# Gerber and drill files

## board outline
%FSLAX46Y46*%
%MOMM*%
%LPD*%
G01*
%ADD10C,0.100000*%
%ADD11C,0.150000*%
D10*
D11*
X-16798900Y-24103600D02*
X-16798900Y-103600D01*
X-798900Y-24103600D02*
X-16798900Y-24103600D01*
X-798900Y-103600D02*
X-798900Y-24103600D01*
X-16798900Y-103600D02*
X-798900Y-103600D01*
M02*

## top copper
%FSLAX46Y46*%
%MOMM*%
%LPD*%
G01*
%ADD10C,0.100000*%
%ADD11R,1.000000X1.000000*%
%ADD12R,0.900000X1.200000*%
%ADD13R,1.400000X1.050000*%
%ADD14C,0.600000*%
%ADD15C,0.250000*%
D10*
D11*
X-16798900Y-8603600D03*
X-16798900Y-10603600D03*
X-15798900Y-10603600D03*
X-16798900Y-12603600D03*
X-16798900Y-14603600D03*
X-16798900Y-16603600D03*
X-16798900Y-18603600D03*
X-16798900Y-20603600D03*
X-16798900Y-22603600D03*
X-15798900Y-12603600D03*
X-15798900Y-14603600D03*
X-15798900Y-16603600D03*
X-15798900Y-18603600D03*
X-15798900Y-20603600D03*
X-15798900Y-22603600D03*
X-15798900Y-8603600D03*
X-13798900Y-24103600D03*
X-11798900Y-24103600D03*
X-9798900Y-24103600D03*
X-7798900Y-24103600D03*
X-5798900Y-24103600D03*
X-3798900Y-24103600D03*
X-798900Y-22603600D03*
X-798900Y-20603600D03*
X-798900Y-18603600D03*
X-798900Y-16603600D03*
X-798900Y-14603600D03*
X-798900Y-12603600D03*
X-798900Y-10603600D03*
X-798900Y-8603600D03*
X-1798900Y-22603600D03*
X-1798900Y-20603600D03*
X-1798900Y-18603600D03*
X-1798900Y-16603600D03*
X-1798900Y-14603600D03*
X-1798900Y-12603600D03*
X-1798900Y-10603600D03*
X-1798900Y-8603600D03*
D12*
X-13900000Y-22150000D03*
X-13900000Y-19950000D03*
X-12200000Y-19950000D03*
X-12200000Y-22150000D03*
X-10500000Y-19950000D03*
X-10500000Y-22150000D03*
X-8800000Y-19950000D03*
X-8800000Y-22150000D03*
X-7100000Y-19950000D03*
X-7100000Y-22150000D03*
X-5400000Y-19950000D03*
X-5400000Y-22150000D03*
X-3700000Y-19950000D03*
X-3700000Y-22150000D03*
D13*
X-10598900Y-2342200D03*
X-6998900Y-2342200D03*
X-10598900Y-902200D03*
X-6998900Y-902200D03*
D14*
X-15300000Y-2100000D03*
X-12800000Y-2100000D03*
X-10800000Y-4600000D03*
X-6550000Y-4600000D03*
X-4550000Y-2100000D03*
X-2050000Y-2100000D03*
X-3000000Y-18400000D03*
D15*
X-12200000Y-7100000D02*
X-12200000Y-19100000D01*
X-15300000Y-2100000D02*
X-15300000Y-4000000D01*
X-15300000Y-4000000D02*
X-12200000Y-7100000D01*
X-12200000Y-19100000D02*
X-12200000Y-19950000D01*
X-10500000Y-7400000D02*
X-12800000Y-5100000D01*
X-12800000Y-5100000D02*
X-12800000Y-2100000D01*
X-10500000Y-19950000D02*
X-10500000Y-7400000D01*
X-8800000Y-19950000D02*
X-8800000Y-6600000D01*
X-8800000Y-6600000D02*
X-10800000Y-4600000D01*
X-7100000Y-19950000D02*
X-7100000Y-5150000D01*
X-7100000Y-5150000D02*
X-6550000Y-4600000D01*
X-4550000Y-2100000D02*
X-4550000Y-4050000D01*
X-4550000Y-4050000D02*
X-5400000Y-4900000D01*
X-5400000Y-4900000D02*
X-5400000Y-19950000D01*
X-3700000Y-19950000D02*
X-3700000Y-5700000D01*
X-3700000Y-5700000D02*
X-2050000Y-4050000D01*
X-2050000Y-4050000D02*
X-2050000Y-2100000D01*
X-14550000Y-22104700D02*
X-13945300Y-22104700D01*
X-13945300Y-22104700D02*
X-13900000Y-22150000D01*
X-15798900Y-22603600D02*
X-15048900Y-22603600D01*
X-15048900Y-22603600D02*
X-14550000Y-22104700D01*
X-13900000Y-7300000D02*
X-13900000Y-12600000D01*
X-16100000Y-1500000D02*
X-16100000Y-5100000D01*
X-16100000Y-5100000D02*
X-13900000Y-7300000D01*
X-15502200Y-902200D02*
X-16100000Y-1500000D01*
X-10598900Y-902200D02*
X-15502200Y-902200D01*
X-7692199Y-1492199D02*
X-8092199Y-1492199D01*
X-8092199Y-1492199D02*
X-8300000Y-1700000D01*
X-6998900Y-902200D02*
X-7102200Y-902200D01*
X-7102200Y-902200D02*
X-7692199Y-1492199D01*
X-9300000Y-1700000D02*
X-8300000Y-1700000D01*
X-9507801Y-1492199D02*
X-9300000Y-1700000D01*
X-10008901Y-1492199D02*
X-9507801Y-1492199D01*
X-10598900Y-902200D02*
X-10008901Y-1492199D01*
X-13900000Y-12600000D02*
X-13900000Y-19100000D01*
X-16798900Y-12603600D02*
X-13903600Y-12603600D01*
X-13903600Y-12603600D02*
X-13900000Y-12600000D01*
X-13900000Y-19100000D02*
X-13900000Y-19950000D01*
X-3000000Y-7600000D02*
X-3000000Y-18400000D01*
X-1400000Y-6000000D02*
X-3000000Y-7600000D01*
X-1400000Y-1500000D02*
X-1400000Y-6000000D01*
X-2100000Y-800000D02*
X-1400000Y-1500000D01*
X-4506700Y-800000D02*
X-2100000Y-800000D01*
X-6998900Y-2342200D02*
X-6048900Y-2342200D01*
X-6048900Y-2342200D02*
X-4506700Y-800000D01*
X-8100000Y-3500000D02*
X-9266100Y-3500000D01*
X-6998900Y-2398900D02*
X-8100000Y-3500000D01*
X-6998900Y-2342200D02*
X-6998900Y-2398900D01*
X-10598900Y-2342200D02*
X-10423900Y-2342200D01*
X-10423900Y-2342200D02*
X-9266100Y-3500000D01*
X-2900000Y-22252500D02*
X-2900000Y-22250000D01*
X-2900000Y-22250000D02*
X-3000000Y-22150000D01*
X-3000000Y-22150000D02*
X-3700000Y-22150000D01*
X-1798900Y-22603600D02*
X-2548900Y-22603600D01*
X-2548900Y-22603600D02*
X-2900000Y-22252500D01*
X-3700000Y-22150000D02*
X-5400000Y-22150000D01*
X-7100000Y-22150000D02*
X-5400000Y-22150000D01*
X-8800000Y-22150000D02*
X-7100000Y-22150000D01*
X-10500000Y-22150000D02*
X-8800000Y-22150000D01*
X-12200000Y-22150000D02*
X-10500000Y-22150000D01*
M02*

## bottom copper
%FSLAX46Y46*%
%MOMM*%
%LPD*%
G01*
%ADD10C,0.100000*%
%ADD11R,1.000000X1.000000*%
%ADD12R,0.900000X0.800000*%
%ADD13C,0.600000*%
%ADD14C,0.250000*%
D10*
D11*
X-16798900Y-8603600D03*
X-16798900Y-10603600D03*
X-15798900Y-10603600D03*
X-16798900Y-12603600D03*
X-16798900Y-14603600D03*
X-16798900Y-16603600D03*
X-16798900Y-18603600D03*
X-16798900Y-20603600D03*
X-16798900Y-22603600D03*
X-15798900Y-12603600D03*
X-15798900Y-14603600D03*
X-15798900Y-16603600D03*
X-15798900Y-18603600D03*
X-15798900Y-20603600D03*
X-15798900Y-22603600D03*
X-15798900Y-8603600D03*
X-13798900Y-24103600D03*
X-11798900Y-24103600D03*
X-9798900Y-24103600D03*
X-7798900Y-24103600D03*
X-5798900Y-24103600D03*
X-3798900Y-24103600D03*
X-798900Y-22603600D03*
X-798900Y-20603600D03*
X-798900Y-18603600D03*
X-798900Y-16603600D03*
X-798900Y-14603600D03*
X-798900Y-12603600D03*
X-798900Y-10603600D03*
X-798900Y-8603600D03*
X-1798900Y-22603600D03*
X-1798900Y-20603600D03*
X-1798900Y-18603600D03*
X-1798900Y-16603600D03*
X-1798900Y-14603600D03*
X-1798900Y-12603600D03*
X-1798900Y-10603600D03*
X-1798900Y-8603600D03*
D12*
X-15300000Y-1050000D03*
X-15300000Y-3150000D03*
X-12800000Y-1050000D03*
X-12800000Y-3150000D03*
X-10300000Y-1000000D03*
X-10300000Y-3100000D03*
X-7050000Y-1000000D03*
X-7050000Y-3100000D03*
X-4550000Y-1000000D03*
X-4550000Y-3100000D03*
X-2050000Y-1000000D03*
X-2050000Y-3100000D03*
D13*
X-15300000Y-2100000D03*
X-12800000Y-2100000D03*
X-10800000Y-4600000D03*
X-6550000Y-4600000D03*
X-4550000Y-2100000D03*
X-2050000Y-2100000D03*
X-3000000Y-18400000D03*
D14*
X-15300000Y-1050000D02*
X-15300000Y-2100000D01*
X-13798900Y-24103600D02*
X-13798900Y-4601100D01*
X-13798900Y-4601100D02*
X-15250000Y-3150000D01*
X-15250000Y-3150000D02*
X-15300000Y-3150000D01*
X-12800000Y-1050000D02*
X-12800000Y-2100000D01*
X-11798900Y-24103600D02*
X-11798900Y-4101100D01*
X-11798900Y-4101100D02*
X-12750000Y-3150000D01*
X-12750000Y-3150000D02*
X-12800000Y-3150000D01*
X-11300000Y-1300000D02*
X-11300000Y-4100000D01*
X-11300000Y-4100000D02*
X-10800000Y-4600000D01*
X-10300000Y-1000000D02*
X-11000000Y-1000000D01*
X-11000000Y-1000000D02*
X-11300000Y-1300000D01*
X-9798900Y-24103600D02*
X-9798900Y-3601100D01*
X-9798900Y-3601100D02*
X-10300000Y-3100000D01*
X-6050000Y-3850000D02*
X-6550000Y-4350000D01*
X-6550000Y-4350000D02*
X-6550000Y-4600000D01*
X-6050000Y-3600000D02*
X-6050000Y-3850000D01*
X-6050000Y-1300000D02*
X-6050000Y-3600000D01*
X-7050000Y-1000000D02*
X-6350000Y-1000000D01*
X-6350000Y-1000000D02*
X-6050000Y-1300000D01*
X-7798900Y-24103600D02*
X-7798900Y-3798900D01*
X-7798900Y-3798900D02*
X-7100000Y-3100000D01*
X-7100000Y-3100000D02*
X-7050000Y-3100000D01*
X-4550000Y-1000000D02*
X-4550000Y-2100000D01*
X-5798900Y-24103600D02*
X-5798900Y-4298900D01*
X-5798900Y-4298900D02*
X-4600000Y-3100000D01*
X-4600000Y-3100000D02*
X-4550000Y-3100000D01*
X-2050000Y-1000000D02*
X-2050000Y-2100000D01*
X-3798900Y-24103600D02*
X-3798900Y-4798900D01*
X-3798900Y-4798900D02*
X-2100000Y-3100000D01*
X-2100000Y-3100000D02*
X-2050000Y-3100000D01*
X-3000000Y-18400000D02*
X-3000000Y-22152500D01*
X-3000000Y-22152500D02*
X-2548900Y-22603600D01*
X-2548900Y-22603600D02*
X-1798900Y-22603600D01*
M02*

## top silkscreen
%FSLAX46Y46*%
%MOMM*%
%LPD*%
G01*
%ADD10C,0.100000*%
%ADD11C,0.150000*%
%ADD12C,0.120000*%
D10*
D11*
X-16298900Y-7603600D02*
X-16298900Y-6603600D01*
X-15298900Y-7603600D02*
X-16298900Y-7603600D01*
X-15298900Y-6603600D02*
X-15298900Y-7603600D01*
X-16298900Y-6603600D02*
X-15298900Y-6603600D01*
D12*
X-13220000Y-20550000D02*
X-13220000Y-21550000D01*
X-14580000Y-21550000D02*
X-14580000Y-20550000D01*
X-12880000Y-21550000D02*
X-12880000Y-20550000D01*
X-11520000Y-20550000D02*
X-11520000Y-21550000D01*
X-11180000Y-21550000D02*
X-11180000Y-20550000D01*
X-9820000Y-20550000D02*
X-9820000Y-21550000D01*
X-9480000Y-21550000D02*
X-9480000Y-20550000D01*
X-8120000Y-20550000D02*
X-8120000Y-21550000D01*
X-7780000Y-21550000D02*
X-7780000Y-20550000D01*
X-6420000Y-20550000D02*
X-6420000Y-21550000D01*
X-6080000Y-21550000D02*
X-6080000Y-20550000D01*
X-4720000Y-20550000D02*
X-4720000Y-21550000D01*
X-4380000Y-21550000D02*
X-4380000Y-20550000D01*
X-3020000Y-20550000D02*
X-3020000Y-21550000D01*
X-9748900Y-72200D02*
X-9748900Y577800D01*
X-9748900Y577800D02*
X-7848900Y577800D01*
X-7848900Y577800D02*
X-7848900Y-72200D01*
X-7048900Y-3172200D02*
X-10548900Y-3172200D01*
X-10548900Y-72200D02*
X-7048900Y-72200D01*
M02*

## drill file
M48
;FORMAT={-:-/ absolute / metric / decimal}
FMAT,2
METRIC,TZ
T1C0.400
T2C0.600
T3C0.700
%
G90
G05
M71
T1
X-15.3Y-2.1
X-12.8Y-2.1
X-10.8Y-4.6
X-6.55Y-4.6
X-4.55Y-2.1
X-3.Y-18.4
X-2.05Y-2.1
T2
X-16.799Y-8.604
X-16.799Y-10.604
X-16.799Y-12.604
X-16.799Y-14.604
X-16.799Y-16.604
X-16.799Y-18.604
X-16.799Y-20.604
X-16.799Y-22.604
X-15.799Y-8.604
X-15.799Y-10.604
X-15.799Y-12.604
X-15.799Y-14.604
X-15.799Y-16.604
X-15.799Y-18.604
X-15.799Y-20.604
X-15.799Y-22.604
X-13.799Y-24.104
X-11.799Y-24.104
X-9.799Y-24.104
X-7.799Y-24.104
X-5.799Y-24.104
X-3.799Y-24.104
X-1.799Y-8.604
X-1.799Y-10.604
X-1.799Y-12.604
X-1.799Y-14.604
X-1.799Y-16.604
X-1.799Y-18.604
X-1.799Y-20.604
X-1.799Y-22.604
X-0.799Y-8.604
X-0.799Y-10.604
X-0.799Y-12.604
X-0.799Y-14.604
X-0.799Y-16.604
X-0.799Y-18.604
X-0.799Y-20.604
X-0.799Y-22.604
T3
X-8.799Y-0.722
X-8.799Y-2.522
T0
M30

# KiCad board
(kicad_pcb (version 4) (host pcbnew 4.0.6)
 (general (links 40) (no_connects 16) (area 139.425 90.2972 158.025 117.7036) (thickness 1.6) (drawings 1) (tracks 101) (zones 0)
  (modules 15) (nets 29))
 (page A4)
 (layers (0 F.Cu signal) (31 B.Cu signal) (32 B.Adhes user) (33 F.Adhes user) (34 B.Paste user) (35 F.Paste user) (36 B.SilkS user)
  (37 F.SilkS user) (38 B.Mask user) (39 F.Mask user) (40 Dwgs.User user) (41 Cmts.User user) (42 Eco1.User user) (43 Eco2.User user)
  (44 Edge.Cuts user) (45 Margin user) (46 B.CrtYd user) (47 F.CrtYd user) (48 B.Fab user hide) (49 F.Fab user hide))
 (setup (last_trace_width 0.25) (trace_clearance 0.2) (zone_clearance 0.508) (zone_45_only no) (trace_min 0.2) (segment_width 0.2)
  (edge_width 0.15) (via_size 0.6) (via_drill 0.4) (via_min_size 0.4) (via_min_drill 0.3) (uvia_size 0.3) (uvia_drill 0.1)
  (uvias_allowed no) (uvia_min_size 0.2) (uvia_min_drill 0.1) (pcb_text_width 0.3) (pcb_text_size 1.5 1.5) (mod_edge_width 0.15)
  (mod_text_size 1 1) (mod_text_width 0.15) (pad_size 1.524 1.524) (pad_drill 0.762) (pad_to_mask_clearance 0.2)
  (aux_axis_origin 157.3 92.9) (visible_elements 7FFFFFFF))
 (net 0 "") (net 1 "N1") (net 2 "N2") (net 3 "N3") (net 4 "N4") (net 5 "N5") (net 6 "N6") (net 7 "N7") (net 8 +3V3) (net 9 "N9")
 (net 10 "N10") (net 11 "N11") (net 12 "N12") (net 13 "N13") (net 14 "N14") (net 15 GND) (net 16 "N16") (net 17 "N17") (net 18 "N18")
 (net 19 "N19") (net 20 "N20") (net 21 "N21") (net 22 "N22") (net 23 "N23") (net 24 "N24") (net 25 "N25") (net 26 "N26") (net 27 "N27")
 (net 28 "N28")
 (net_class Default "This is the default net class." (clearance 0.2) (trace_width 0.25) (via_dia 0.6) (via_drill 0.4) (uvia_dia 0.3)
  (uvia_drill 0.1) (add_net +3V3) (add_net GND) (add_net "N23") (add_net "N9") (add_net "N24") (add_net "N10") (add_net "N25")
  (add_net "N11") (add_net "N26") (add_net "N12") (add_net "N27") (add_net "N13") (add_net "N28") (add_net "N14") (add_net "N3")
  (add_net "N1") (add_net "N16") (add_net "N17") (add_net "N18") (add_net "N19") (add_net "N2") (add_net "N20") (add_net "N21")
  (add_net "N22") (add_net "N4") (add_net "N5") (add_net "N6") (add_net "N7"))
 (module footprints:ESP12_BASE (layer F.Cu) (at 148.5011 105.0036)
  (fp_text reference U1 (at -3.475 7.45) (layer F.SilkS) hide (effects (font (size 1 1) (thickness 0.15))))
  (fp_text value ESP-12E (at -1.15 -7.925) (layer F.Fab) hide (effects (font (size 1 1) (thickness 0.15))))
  (fp_line (start -7.5 -4.5) (end -7.5 -5.5) (layer F.SilkS) (width 0.15))
  (fp_line (start -6.5 -4.5) (end -7.5 -4.5) (layer F.SilkS) (width 0.15))
  (fp_line (start -6.5 -5.5) (end -6.5 -4.5) (layer F.SilkS) (width 0.15))
  (fp_line (start -7.5 -5.5) (end -6.5 -5.5) (layer F.SilkS) (width 0.15))
  (fp_line (start -8 12) (end -8 -12) (layer Edge.Cuts) (width 0.15))
  (fp_line (start 8 12) (end -8 12) (layer Edge.Cuts) (width 0.15))
  (fp_line (start 8 -12) (end 8 12) (layer Edge.Cuts) (width 0.15))
  (fp_line (start -8 -12) (end 8 -12) (layer Edge.Cuts) (width 0.15))
  (pad 1 thru_hole rect (at -8 -3.5) (size 1 1) (drill 0.6) (layers *.Cu *.Mask) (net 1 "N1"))
  (pad 2 thru_hole rect (at -8 -1.5) (size 1 1) (drill 0.6) (layers *.Cu *.Mask) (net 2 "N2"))
  (pad 2 thru_hole rect (at -7 -1.5) (size 1 1) (drill 0.6) (layers *.Cu *.Mask) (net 2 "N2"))
  (pad 3 thru_hole rect (at -8 0.5) (size 1 1) (drill 0.6) (layers *.Cu *.Mask) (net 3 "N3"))
  (pad 4 thru_hole rect (at -8 2.5) (size 1 1) (drill 0.6) (layers *.Cu *.Mask) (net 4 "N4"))
  (pad 5 thru_hole rect (at -8 4.5) (size 1 1) (drill 0.6) (layers *.Cu *.Mask) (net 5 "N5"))
  (pad 6 thru_hole rect (at -8 6.5) (size 1 1) (drill 0.6) (layers *.Cu *.Mask) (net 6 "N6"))
  (pad 7 thru_hole rect (at -8 8.5) (size 1 1) (drill 0.6) (layers *.Cu *.Mask) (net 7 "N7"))
  (pad 8 thru_hole rect (at -8 10.5) (size 1 1) (drill 0.6) (layers *.Cu *.Mask) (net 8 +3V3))
  (pad 3 thru_hole rect (at -7 0.5) (size 1 1) (drill 0.6) (layers *.Cu *.Mask) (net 3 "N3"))
  (pad 4 thru_hole rect (at -7 2.5) (size 1 1) (drill 0.6) (layers *.Cu *.Mask) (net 4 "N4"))
  (pad 5 thru_hole rect (at -7 4.5) (size 1 1) (drill 0.6) (layers *.Cu *.Mask) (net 5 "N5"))
  (pad 6 thru_hole rect (at -7 6.5) (size 1 1) (drill 0.6) (layers *.Cu *.Mask) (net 6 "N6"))
  (pad 7 thru_hole rect (at -7 8.5) (size 1 1) (drill 0.6) (layers *.Cu *.Mask) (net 7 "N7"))
  (pad 8 thru_hole rect (at -7 10.5) (size 1 1) (drill 0.6) (layers *.Cu *.Mask) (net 8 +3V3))
  (pad 1 thru_hole rect (at -7 -3.5) (size 1 1) (drill 0.6) (layers *.Cu *.Mask) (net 1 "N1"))
  (pad 9 thru_hole rect (at -5 12) (size 1 1) (drill 0.6) (layers *.Cu *.Mask) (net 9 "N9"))
  (pad 10 thru_hole rect (at -3 12) (size 1 1) (drill 0.6) (layers *.Cu *.Mask) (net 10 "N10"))
  (pad 11 thru_hole rect (at -1 12) (size 1 1) (drill 0.6) (layers *.Cu *.Mask) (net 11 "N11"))
  (pad 12 thru_hole rect (at 1 12) (size 1 1) (drill 0.6) (layers *.Cu *.Mask) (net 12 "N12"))
  (pad 13 thru_hole rect (at 3 12) (size 1 1) (drill 0.6) (layers *.Cu *.Mask) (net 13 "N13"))
  (pad 14 thru_hole rect (at 5 12) (size 1 1) (drill 0.6) (layers *.Cu *.Mask) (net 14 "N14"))
  (pad 15 thru_hole rect (at 8 10.5) (size 1 1) (drill 0.6) (layers *.Cu *.Mask) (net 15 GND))
  (pad 16 thru_hole rect (at 8 8.5) (size 1 1) (drill 0.6) (layers *.Cu *.Mask) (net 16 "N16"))
  (pad 17 thru_hole rect (at 8 6.5) (size 1 1) (drill 0.6) (layers *.Cu *.Mask) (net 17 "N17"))
  (pad 18 thru_hole rect (at 8 4.5) (size 1 1) (drill 0.6) (layers *.Cu *.Mask) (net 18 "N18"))
  (pad 19 thru_hole rect (at 8 2.5) (size 1 1) (drill 0.6) (layers *.Cu *.Mask) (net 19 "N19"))
  (pad 20 thru_hole rect (at 8 0.5) (size 1 1) (drill 0.6) (layers *.Cu *.Mask) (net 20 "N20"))
  (pad 21 thru_hole rect (at 8 -1.5) (size 1 1) (drill 0.6) (layers *.Cu *.Mask) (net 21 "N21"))
  (pad 22 thru_hole rect (at 8 -3.5) (size 1 1) (drill 0.6) (layers *.Cu *.Mask) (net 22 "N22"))
  (pad 15 thru_hole rect (at 7 10.5) (size 1 1) (drill 0.6) (layers *.Cu *.Mask) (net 15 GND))
  (pad 16 thru_hole rect (at 7 8.5) (size 1 1) (drill 0.6) (layers *.Cu *.Mask) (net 16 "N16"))
  (pad 17 thru_hole rect (at 7 6.5) (size 1 1) (drill 0.6) (layers *.Cu *.Mask) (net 17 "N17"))
  (pad 18 thru_hole rect (at 7 4.5) (size 1 1) (drill 0.6) (layers *.Cu *.Mask) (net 18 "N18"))
  (pad 19 thru_hole rect (at 7 2.5) (size 1 1) (drill 0.6) (layers *.Cu *.Mask) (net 19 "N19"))
  (pad 20 thru_hole rect (at 7 0.5) (size 1 1) (drill 0.6) (layers *.Cu *.Mask) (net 20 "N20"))
  (pad 21 thru_hole rect (at 7 -1.5) (size 1 1) (drill 0.6) (layers *.Cu *.Mask) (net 21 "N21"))
  (pad 22 thru_hole rect (at 7 -3.5) (size 1 1) (drill 0.6) (layers *.Cu *.Mask) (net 22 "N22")))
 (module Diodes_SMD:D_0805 (layer B.Cu) (at 142 95 270)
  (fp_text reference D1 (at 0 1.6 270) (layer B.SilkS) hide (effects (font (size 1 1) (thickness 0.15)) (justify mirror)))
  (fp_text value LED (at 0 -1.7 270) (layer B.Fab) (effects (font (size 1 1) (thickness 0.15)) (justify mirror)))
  (pad 1 smd rect (at -1.05 0 270) (size 0.8 0.9) (layers B.Cu B.Paste B.Mask) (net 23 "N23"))
  (pad 2 smd rect (at 1.05 0 270) (size 0.8 0.9) (layers B.Cu B.Paste B.Mask) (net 9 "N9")))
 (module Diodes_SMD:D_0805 (layer B.Cu) (at 144.5 95 270)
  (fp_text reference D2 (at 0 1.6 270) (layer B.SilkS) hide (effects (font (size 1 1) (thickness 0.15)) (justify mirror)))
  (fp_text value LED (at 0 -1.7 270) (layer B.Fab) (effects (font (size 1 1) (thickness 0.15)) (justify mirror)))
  (pad 1 smd rect (at -1.05 0 270) (size 0.8 0.9) (layers B.Cu B.Paste B.Mask) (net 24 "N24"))
  (pad 2 smd rect (at 1.05 0 270) (size 0.8 0.9) (layers B.Cu B.Paste B.Mask) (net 10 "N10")))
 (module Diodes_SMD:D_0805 (layer B.Cu) (at 147 94.95 270)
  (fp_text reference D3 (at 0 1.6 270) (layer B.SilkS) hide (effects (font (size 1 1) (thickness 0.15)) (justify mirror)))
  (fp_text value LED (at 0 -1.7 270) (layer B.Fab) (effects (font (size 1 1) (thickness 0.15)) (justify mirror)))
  (pad 1 smd rect (at -1.05 0 270) (size 0.8 0.9) (layers B.Cu B.Paste B.Mask) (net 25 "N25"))
  (pad 2 smd rect (at 1.05 0 270) (size 0.8 0.9) (layers B.Cu B.Paste B.Mask) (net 11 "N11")))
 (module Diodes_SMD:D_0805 (layer B.Cu) (at 150.25 94.95 270)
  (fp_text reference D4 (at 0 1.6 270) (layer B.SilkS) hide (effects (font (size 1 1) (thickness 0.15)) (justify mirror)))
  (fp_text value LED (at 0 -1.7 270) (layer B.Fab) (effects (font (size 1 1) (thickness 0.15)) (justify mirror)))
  (pad 1 smd rect (at -1.05 0 270) (size 0.8 0.9) (layers B.Cu B.Paste B.Mask) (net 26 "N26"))
  (pad 2 smd rect (at 1.05 0 270) (size 0.8 0.9) (layers B.Cu B.Paste B.Mask) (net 12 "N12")))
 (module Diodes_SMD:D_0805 (layer B.Cu) (at 152.75 94.95 270)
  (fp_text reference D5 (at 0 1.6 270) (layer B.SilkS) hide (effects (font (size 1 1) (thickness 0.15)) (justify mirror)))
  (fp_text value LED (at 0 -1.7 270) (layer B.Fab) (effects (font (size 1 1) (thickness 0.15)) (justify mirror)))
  (pad 1 smd rect (at -1.05 0 270) (size 0.8 0.9) (layers B.Cu B.Paste B.Mask) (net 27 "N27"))
  (pad 2 smd rect (at 1.05 0 270) (size 0.8 0.9) (layers B.Cu B.Paste B.Mask) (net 13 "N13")))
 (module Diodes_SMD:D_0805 (layer B.Cu) (at 155.25 94.95 270)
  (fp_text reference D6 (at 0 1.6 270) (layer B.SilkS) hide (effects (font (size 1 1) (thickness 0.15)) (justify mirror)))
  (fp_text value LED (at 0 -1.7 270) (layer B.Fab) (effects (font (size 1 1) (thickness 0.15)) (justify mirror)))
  (pad 1 smd rect (at -1.05 0 270) (size 0.8 0.9) (layers B.Cu B.Paste B.Mask) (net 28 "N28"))
  (pad 2 smd rect (at 1.05 0 270) (size 0.8 0.9) (layers B.Cu B.Paste B.Mask) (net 14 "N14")))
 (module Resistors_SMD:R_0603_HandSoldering (layer F.Cu) (at 143.4 113.95 90)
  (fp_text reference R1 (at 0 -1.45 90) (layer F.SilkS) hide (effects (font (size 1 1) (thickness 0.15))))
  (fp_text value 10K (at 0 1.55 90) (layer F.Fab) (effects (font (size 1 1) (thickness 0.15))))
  (fp_line (start 0.5 0.68) (end -0.5 0.68) (layer F.SilkS) (width 0.12))
  (fp_line (start -0.5 -0.68) (end 0.5 -0.68) (layer F.SilkS) (width 0.12))
  (pad 1 smd rect (at -1.1 0 90) (size 1.2 0.9) (layers F.Cu F.Paste F.Mask) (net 8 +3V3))
  (pad 2 smd rect (at 1.1 0 90) (size 1.2 0.9) (layers F.Cu F.Paste F.Mask) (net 3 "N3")))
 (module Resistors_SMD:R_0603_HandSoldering (layer F.Cu) (at 145.1 113.95 270)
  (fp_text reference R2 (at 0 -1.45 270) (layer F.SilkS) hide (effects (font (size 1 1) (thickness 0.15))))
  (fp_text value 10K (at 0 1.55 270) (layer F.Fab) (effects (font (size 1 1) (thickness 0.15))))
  (fp_line (start 0.5 0.68) (end -0.5 0.68) (layer F.SilkS) (width 0.12))
  (fp_line (start -0.5 -0.68) (end 0.5 -0.68) (layer F.SilkS) (width 0.12))
  (pad 1 smd rect (at -1.1 0 270) (size 1.2 0.9) (layers F.Cu F.Paste F.Mask) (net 23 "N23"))
  (pad 2 smd rect (at 1.1 0 270) (size 1.2 0.9) (layers F.Cu F.Paste F.Mask) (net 15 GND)))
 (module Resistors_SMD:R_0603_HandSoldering (layer F.Cu) (at 146.8 113.95 270)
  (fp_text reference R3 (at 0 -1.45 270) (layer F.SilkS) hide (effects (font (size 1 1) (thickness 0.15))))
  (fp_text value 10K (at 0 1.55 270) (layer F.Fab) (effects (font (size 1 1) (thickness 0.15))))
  (fp_line (start 0.5 0.68) (end -0.5 0.68) (layer F.SilkS) (width 0.12))
  (fp_line (start -0.5 -0.68) (end 0.5 -0.68) (layer F.SilkS) (width 0.12))
  (pad 1 smd rect (at -1.1 0 270) (size 1.2 0.9) (layers F.Cu F.Paste F.Mask) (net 24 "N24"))
  (pad 2 smd rect (at 1.1 0 270) (size 1.2 0.9) (layers F.Cu F.Paste F.Mask) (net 15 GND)))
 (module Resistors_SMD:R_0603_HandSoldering (layer F.Cu) (at 148.5 113.95 270)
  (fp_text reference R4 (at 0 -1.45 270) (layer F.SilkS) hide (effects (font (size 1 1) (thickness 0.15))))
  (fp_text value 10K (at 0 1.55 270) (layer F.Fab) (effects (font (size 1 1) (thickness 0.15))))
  (fp_line (start 0.5 0.68) (end -0.5 0.68) (layer F.SilkS) (width 0.12))
  (fp_line (start -0.5 -0.68) (end 0.5 -0.68) (layer F.SilkS) (width 0.12))
  (pad 1 smd rect (at -1.1 0 270) (size 1.2 0.9) (layers F.Cu F.Paste F.Mask) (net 25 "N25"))
  (pad 2 smd rect (at 1.1 0 270) (size 1.2 0.9) (layers F.Cu F.Paste F.Mask) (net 15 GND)))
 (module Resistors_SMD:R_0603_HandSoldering (layer F.Cu) (at 150.2 113.95 270)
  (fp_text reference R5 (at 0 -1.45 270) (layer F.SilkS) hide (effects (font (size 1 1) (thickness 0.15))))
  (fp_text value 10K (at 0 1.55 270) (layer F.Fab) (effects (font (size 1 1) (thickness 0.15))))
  (fp_line (start 0.5 0.68) (end -0.5 0.68) (layer F.SilkS) (width 0.12))
  (fp_line (start -0.5 -0.68) (end 0.5 -0.68) (layer F.SilkS) (width 0.12))
  (pad 1 smd rect (at -1.1 0 270) (size 1.2 0.9) (layers F.Cu F.Paste F.Mask) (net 26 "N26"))
  (pad 2 smd rect (at 1.1 0 270) (size 1.2 0.9) (layers F.Cu F.Paste F.Mask) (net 15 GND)))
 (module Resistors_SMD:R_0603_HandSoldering (layer F.Cu) (at 151.9 113.95 270)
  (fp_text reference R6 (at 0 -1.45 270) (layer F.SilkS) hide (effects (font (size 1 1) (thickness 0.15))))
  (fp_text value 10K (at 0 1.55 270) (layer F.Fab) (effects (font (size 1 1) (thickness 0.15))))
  (fp_line (start 0.5 0.68) (end -0.5 0.68) (layer F.SilkS) (width 0.12))
  (fp_line (start -0.5 -0.68) (end 0.5 -0.68) (layer F.SilkS) (width 0.12))
  (pad 1 smd rect (at -1.1 0 270) (size 1.2 0.9) (layers F.Cu F.Paste F.Mask) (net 27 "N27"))
  (pad 2 smd rect (at 1.1 0 270) (size 1.2 0.9) (layers F.Cu F.Paste F.Mask) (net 15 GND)))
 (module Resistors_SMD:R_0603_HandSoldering (layer F.Cu) (at 153.6 113.95 270)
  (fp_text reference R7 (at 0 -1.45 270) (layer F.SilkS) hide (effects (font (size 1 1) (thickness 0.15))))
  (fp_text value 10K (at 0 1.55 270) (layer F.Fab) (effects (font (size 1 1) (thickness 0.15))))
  (fp_line (start 0.5 0.68) (end -0.5 0.68) (layer F.SilkS) (width 0.12))
  (fp_line (start -0.5 -0.68) (end 0.5 -0.68) (layer F.SilkS) (width 0.12))
  (pad 1 smd rect (at -1.1 0 270) (size 1.2 0.9) (layers F.Cu F.Paste F.Mask) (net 28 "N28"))
  (pad 2 smd rect (at 1.1 0 270) (size 1.2 0.9) (layers F.Cu F.Paste F.Mask) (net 15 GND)))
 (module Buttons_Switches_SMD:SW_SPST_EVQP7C (layer F.Cu) (at 148.5011 94.5222 180)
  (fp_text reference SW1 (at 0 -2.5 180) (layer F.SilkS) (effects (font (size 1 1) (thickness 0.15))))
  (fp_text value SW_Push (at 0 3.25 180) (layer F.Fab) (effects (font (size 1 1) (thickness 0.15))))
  (fp_line (start 0.95 1.55) (end 0.95 2.2) (layer F.SilkS) (width 0.12))
  (fp_line (start 0.95 2.2) (end -0.95 2.2) (layer F.SilkS) (width 0.12))
  (fp_line (start -0.95 2.2) (end -0.95 1.55) (layer F.SilkS) (width 0.12))
  (fp_line (start -1.75 -1.55) (end 1.75 -1.55) (layer F.SilkS) (width 0.12))
  (fp_line (start 1.75 1.55) (end -1.75 1.55) (layer F.SilkS) (width 0.12))
  (pad 1 smd rect (at 1.8 -0.72 180) (size 1.4 1.05) (layers F.Cu F.Paste F.Mask) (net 15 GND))
  (pad 1 smd rect (at -1.8 -0.72 180) (size 1.4 1.05) (layers F.Cu F.Paste F.Mask) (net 15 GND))
  (pad 2 smd rect (at 1.8 0.72 180) (size 1.4 1.05) (layers F.Cu F.Paste F.Mask) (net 3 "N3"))
  (pad 2 smd rect (at -1.8 0.72 180) (size 1.4 1.05) (layers F.Cu F.Paste F.Mask) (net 3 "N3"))
  (pad "" np_thru_hole circle (at 0 -0.9 180) (size 0.7 0.7) (drill 0.7) (layers *.Cu *.Mask))
  (pad "" np_thru_hole circle (at 0 0.9 180) (size 0.7 0.7) (drill 0.7) (layers *.Cu *.Mask)))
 (segment (start 145.1 100) (end 145.1 112) (width 0.25) (layer F.Cu) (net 23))
 (segment (start 142 95) (end 142 96.9) (width 0.25) (layer F.Cu) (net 23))
 (segment (start 142 96.9) (end 145.1 100) (width 0.25) (layer F.Cu) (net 23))
 (segment (start 145.1 112) (end 145.1 112.85) (width 0.25) (layer F.Cu) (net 23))
 (segment (start 142 93.95) (end 142 95) (width 0.25) (layer B.Cu) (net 23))
 (via (at 142 95) (size 0.6) (drill 0.4) (layers F.Cu B.Cu) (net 23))
 (segment (start 143.5011 117.0036) (end 143.5011 97.5011) (width 0.25) (layer B.Cu) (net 9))
 (segment (start 143.5011 97.5011) (end 142.05 96.05) (width 0.25) (layer B.Cu) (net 9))
 (segment (start 142.05 96.05) (end 142 96.05) (width 0.25) (layer B.Cu) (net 9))
 (segment (start 146.8 100.3) (end 144.5 98) (width 0.25) (layer F.Cu) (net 24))
 (segment (start 144.5 98) (end 144.5 95) (width 0.25) (layer F.Cu) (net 24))
 (segment (start 146.8 112.85) (end 146.8 100.3) (width 0.25) (layer F.Cu) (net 24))
 (segment (start 144.5 93.95) (end 144.5 95) (width 0.25) (layer B.Cu) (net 24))
 (via (at 144.5 95) (size 0.6) (drill 0.4) (layers F.Cu B.Cu) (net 24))
 (segment (start 145.5011 117.0036) (end 145.5011 97.0011) (width 0.25) (layer B.Cu) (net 10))
 (segment (start 145.5011 97.0011) (end 144.55 96.05) (width 0.25) (layer B.Cu) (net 10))
 (segment (start 144.55 96.05) (end 144.5 96.05) (width 0.25) (layer B.Cu) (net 10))
 (segment (start 148.5 112.85) (end 148.5 99.5) (width 0.25) (layer F.Cu) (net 25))
 (segment (start 148.5 99.5) (end 146.5 97.5) (width 0.25) (layer F.Cu) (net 25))
 (segment (start 146 94.2) (end 146 97) (width 0.25) (layer B.Cu) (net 25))
 (segment (start 146 97) (end 146.5 97.5) (width 0.25) (layer B.Cu) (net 25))
 (via (at 146.5 97.5) (size 0.6) (drill 0.4) (layers F.Cu B.Cu) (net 25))
 (segment (start 147 93.9) (end 146.3 93.9) (width 0.25) (layer B.Cu) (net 25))
 (segment (start 146.3 93.9) (end 146 94.2) (width 0.25) (layer B.Cu) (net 25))
 (segment (start 147.5011 117.0036) (end 147.5011 96.5011) (width 0.25) (layer B.Cu) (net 11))
 (segment (start 147.5011 96.5011) (end 147 96) (width 0.25) (layer B.Cu) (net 11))
 (segment (start 150.2 112.85) (end 150.2 98.05) (width 0.25) (layer F.Cu) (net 26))
 (segment (start 150.2 98.05) (end 150.75 97.5) (width 0.25) (layer F.Cu) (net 26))
 (segment (start 151.25 96.75) (end 150.75 97.25) (width 0.25) (layer B.Cu) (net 26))
 (segment (start 150.75 97.25) (end 150.75 97.5) (width 0.25) (layer B.Cu) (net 26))
 (via (at 150.75 97.5) (size 0.6) (drill 0.4) (layers F.Cu B.Cu) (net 26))
 (segment (start 151.25 96.5) (end 151.25 96.75) (width 0.25) (layer B.Cu) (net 26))
 (segment (start 151.25 94.2) (end 151.25 96.5) (width 0.25) (layer B.Cu) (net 26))
 (segment (start 150.25 93.9) (end 150.95 93.9) (width 0.25) (layer B.Cu) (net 26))
 (segment (start 150.95 93.9) (end 151.25 94.2) (width 0.25) (layer B.Cu) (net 26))
 (segment (start 149.5011 117.0036) (end 149.5011 96.6989) (width 0.25) (layer B.Cu) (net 12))
 (segment (start 149.5011 96.6989) (end 150.2 96) (width 0.25) (layer B.Cu) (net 12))
 (segment (start 150.2 96) (end 150.25 96) (width 0.25) (layer B.Cu) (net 12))
 (segment (start 152.75 95) (end 152.75 96.95) (width 0.25) (layer F.Cu) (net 27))
 (segment (start 152.75 96.95) (end 151.9 97.8) (width 0.25) (layer F.Cu) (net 27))
 (segment (start 151.9 97.8) (end 151.9 112.85) (width 0.25) (layer F.Cu) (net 27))
 (segment (start 152.75 93.9) (end 152.75 95) (width 0.25) (layer B.Cu) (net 27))
 (via (at 152.75 95) (size 0.6) (drill 0.4) (layers F.Cu B.Cu) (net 27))
 (segment (start 151.5011 117.0036) (end 151.5011 97.1989) (width 0.25) (layer B.Cu) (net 13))
 (segment (start 151.5011 97.1989) (end 152.7 96) (width 0.25) (layer B.Cu) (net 13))
 (segment (start 152.7 96) (end 152.75 96) (width 0.25) (layer B.Cu) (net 13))
 (segment (start 153.6 112.85) (end 153.6 98.6) (width 0.25) (layer F.Cu) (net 28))
 (segment (start 153.6 98.6) (end 155.25 96.95) (width 0.25) (layer F.Cu) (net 28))
 (segment (start 155.25 96.95) (end 155.25 95) (width 0.25) (layer F.Cu) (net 28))
 (segment (start 155.25 93.9) (end 155.25 95) (width 0.25) (layer B.Cu) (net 28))
 (via (at 155.25 95) (size 0.6) (drill 0.4) (layers F.Cu B.Cu) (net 28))
 (segment (start 153.5011 117.0036) (end 153.5011 97.6989) (width 0.25) (layer B.Cu) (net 14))
 (segment (start 153.5011 97.6989) (end 155.2 96) (width 0.25) (layer B.Cu) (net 14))
 (segment (start 155.2 96) (end 155.25 96) (width 0.25) (layer B.Cu) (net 14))
 (segment (start 142.75 115.0047) (end 143.3547 115.0047) (width 0.25) (layer F.Cu) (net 8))
 (segment (start 143.3547 115.0047) (end 143.4 115.05) (width 0.25) (layer F.Cu) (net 8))
 (segment (start 141.5011 115.5036) (end 142.2511 115.5036) (width 0.25) (layer F.Cu) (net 8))
 (segment (start 142.2511 115.5036) (end 142.75 115.0047) (width 0.25) (layer F.Cu) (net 8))
 (segment (start 143.4 100.2) (end 143.4 105.5) (width 0.25) (layer F.Cu) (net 3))
 (segment (start 141.2 94.4) (end 141.2 98) (width 0.25) (layer F.Cu) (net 3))
 (segment (start 141.2 98) (end 143.4 100.2) (width 0.25) (layer F.Cu) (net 3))
 (segment (start 141.7978 93.8022) (end 141.2 94.4) (width 0.25) (layer F.Cu) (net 3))
 (segment (start 146.7011 93.8022) (end 141.7978 93.8022) (width 0.25) (layer F.Cu) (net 3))
 (segment (start 149.607801 94.392199) (end 149.207801 94.392199) (width 0.25) (layer F.Cu) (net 3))
 (segment (start 149.207801 94.392199) (end 149 94.6) (width 0.25) (layer F.Cu) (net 3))
 (segment (start 150.3011 93.8022) (end 150.1978 93.8022) (width 0.25) (layer F.Cu) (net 3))
 (segment (start 150.1978 93.8022) (end 149.607801 94.392199) (width 0.25) (layer F.Cu) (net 3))
 (segment (start 148 94.6) (end 149 94.6) (width 0.25) (layer F.Cu) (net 3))
 (segment (start 147.792199 94.392199) (end 148 94.6) (width 0.25) (layer F.Cu) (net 3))
 (segment (start 147.291099 94.392199) (end 147.792199 94.392199) (width 0.25) (layer F.Cu) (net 3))
 (segment (start 146.7011 93.8022) (end 147.291099 94.392199) (width 0.25) (layer F.Cu) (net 3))
 (segment (start 143.4 105.5) (end 143.4 112) (width 0.25) (layer F.Cu) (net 3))
 (segment (start 140.5011 105.5036) (end 143.3964 105.5036) (width 0.25) (layer F.Cu) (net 3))
 (segment (start 143.3964 105.5036) (end 143.4 105.5) (width 0.25) (layer F.Cu) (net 3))
 (segment (start 143.4 112) (end 143.4 112.85) (width 0.25) (layer F.Cu) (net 3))
 (segment (start 154.3 111.3) (end 154.3 115.0525) (width 0.25) (layer B.Cu) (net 15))
 (segment (start 154.3 115.0525) (end 154.7511 115.5036) (width 0.25) (layer B.Cu) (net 15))
 (segment (start 154.7511 115.5036) (end 155.5011 115.5036) (width 0.25) (layer B.Cu) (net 15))
 (via (at 154.3 111.3) (size 0.6) (drill 0.4) (layers F.Cu B.Cu) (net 15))
 (segment (start 154.3 100.5) (end 154.3 111.3) (width 0.25) (layer F.Cu) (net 15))
 (segment (start 155.9 98.9) (end 154.3 100.5) (width 0.25) (layer F.Cu) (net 15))
 (segment (start 155.9 94.4) (end 155.9 98.9) (width 0.25) (layer F.Cu) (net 15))
 (segment (start 155.2 93.7) (end 155.9 94.4) (width 0.25) (layer F.Cu) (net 15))
 (segment (start 152.7933 93.7) (end 155.2 93.7) (width 0.25) (layer F.Cu) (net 15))
 (segment (start 150.3011 95.2422) (end 151.2511 95.2422) (width 0.25) (layer F.Cu) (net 15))
 (segment (start 151.2511 95.2422) (end 152.7933 93.7) (width 0.25) (layer F.Cu) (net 15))
 (segment (start 149.2 96.4) (end 148.0339 96.4) (width 0.25) (layer F.Cu) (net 15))
 (segment (start 150.3011 95.2989) (end 149.2 96.4) (width 0.25) (layer F.Cu) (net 15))
 (segment (start 150.3011 95.2422) (end 150.3011 95.2989) (width 0.25) (layer F.Cu) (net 15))
 (segment (start 146.7011 95.2422) (end 146.8761 95.2422) (width 0.25) (layer F.Cu) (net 15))
 (segment (start 146.8761 95.2422) (end 148.0339 96.4) (width 0.25) (layer F.Cu) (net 15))
 (segment (start 154.4 115.1525) (end 154.4 115.15) (width 0.25) (layer F.Cu) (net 15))
 (segment (start 154.4 115.15) (end 154.3 115.05) (width 0.25) (layer F.Cu) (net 15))
 (segment (start 154.3 115.05) (end 153.6 115.05) (width 0.25) (layer F.Cu) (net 15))
 (segment (start 155.5011 115.5036) (end 154.7511 115.5036) (width 0.25) (layer F.Cu) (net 15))
 (segment (start 154.7511 115.5036) (end 154.4 115.1525) (width 0.25) (layer F.Cu) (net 15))
 (segment (start 153.6 115.05) (end 151.9 115.05) (width 0.25) (layer F.Cu) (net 15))
 (segment (start 150.2 115.05) (end 151.9 115.05) (width 0.25) (layer F.Cu) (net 15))
 (segment (start 148.5 115.05) (end 150.2 115.05) (width 0.25) (layer F.Cu) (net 15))
 (segment (start 146.8 115.05) (end 148.5 115.05) (width 0.25) (layer F.Cu) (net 15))
 (segment (start 145.1 115.05) (end 146.8 115.05) (width 0.25) (layer F.Cu) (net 15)))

